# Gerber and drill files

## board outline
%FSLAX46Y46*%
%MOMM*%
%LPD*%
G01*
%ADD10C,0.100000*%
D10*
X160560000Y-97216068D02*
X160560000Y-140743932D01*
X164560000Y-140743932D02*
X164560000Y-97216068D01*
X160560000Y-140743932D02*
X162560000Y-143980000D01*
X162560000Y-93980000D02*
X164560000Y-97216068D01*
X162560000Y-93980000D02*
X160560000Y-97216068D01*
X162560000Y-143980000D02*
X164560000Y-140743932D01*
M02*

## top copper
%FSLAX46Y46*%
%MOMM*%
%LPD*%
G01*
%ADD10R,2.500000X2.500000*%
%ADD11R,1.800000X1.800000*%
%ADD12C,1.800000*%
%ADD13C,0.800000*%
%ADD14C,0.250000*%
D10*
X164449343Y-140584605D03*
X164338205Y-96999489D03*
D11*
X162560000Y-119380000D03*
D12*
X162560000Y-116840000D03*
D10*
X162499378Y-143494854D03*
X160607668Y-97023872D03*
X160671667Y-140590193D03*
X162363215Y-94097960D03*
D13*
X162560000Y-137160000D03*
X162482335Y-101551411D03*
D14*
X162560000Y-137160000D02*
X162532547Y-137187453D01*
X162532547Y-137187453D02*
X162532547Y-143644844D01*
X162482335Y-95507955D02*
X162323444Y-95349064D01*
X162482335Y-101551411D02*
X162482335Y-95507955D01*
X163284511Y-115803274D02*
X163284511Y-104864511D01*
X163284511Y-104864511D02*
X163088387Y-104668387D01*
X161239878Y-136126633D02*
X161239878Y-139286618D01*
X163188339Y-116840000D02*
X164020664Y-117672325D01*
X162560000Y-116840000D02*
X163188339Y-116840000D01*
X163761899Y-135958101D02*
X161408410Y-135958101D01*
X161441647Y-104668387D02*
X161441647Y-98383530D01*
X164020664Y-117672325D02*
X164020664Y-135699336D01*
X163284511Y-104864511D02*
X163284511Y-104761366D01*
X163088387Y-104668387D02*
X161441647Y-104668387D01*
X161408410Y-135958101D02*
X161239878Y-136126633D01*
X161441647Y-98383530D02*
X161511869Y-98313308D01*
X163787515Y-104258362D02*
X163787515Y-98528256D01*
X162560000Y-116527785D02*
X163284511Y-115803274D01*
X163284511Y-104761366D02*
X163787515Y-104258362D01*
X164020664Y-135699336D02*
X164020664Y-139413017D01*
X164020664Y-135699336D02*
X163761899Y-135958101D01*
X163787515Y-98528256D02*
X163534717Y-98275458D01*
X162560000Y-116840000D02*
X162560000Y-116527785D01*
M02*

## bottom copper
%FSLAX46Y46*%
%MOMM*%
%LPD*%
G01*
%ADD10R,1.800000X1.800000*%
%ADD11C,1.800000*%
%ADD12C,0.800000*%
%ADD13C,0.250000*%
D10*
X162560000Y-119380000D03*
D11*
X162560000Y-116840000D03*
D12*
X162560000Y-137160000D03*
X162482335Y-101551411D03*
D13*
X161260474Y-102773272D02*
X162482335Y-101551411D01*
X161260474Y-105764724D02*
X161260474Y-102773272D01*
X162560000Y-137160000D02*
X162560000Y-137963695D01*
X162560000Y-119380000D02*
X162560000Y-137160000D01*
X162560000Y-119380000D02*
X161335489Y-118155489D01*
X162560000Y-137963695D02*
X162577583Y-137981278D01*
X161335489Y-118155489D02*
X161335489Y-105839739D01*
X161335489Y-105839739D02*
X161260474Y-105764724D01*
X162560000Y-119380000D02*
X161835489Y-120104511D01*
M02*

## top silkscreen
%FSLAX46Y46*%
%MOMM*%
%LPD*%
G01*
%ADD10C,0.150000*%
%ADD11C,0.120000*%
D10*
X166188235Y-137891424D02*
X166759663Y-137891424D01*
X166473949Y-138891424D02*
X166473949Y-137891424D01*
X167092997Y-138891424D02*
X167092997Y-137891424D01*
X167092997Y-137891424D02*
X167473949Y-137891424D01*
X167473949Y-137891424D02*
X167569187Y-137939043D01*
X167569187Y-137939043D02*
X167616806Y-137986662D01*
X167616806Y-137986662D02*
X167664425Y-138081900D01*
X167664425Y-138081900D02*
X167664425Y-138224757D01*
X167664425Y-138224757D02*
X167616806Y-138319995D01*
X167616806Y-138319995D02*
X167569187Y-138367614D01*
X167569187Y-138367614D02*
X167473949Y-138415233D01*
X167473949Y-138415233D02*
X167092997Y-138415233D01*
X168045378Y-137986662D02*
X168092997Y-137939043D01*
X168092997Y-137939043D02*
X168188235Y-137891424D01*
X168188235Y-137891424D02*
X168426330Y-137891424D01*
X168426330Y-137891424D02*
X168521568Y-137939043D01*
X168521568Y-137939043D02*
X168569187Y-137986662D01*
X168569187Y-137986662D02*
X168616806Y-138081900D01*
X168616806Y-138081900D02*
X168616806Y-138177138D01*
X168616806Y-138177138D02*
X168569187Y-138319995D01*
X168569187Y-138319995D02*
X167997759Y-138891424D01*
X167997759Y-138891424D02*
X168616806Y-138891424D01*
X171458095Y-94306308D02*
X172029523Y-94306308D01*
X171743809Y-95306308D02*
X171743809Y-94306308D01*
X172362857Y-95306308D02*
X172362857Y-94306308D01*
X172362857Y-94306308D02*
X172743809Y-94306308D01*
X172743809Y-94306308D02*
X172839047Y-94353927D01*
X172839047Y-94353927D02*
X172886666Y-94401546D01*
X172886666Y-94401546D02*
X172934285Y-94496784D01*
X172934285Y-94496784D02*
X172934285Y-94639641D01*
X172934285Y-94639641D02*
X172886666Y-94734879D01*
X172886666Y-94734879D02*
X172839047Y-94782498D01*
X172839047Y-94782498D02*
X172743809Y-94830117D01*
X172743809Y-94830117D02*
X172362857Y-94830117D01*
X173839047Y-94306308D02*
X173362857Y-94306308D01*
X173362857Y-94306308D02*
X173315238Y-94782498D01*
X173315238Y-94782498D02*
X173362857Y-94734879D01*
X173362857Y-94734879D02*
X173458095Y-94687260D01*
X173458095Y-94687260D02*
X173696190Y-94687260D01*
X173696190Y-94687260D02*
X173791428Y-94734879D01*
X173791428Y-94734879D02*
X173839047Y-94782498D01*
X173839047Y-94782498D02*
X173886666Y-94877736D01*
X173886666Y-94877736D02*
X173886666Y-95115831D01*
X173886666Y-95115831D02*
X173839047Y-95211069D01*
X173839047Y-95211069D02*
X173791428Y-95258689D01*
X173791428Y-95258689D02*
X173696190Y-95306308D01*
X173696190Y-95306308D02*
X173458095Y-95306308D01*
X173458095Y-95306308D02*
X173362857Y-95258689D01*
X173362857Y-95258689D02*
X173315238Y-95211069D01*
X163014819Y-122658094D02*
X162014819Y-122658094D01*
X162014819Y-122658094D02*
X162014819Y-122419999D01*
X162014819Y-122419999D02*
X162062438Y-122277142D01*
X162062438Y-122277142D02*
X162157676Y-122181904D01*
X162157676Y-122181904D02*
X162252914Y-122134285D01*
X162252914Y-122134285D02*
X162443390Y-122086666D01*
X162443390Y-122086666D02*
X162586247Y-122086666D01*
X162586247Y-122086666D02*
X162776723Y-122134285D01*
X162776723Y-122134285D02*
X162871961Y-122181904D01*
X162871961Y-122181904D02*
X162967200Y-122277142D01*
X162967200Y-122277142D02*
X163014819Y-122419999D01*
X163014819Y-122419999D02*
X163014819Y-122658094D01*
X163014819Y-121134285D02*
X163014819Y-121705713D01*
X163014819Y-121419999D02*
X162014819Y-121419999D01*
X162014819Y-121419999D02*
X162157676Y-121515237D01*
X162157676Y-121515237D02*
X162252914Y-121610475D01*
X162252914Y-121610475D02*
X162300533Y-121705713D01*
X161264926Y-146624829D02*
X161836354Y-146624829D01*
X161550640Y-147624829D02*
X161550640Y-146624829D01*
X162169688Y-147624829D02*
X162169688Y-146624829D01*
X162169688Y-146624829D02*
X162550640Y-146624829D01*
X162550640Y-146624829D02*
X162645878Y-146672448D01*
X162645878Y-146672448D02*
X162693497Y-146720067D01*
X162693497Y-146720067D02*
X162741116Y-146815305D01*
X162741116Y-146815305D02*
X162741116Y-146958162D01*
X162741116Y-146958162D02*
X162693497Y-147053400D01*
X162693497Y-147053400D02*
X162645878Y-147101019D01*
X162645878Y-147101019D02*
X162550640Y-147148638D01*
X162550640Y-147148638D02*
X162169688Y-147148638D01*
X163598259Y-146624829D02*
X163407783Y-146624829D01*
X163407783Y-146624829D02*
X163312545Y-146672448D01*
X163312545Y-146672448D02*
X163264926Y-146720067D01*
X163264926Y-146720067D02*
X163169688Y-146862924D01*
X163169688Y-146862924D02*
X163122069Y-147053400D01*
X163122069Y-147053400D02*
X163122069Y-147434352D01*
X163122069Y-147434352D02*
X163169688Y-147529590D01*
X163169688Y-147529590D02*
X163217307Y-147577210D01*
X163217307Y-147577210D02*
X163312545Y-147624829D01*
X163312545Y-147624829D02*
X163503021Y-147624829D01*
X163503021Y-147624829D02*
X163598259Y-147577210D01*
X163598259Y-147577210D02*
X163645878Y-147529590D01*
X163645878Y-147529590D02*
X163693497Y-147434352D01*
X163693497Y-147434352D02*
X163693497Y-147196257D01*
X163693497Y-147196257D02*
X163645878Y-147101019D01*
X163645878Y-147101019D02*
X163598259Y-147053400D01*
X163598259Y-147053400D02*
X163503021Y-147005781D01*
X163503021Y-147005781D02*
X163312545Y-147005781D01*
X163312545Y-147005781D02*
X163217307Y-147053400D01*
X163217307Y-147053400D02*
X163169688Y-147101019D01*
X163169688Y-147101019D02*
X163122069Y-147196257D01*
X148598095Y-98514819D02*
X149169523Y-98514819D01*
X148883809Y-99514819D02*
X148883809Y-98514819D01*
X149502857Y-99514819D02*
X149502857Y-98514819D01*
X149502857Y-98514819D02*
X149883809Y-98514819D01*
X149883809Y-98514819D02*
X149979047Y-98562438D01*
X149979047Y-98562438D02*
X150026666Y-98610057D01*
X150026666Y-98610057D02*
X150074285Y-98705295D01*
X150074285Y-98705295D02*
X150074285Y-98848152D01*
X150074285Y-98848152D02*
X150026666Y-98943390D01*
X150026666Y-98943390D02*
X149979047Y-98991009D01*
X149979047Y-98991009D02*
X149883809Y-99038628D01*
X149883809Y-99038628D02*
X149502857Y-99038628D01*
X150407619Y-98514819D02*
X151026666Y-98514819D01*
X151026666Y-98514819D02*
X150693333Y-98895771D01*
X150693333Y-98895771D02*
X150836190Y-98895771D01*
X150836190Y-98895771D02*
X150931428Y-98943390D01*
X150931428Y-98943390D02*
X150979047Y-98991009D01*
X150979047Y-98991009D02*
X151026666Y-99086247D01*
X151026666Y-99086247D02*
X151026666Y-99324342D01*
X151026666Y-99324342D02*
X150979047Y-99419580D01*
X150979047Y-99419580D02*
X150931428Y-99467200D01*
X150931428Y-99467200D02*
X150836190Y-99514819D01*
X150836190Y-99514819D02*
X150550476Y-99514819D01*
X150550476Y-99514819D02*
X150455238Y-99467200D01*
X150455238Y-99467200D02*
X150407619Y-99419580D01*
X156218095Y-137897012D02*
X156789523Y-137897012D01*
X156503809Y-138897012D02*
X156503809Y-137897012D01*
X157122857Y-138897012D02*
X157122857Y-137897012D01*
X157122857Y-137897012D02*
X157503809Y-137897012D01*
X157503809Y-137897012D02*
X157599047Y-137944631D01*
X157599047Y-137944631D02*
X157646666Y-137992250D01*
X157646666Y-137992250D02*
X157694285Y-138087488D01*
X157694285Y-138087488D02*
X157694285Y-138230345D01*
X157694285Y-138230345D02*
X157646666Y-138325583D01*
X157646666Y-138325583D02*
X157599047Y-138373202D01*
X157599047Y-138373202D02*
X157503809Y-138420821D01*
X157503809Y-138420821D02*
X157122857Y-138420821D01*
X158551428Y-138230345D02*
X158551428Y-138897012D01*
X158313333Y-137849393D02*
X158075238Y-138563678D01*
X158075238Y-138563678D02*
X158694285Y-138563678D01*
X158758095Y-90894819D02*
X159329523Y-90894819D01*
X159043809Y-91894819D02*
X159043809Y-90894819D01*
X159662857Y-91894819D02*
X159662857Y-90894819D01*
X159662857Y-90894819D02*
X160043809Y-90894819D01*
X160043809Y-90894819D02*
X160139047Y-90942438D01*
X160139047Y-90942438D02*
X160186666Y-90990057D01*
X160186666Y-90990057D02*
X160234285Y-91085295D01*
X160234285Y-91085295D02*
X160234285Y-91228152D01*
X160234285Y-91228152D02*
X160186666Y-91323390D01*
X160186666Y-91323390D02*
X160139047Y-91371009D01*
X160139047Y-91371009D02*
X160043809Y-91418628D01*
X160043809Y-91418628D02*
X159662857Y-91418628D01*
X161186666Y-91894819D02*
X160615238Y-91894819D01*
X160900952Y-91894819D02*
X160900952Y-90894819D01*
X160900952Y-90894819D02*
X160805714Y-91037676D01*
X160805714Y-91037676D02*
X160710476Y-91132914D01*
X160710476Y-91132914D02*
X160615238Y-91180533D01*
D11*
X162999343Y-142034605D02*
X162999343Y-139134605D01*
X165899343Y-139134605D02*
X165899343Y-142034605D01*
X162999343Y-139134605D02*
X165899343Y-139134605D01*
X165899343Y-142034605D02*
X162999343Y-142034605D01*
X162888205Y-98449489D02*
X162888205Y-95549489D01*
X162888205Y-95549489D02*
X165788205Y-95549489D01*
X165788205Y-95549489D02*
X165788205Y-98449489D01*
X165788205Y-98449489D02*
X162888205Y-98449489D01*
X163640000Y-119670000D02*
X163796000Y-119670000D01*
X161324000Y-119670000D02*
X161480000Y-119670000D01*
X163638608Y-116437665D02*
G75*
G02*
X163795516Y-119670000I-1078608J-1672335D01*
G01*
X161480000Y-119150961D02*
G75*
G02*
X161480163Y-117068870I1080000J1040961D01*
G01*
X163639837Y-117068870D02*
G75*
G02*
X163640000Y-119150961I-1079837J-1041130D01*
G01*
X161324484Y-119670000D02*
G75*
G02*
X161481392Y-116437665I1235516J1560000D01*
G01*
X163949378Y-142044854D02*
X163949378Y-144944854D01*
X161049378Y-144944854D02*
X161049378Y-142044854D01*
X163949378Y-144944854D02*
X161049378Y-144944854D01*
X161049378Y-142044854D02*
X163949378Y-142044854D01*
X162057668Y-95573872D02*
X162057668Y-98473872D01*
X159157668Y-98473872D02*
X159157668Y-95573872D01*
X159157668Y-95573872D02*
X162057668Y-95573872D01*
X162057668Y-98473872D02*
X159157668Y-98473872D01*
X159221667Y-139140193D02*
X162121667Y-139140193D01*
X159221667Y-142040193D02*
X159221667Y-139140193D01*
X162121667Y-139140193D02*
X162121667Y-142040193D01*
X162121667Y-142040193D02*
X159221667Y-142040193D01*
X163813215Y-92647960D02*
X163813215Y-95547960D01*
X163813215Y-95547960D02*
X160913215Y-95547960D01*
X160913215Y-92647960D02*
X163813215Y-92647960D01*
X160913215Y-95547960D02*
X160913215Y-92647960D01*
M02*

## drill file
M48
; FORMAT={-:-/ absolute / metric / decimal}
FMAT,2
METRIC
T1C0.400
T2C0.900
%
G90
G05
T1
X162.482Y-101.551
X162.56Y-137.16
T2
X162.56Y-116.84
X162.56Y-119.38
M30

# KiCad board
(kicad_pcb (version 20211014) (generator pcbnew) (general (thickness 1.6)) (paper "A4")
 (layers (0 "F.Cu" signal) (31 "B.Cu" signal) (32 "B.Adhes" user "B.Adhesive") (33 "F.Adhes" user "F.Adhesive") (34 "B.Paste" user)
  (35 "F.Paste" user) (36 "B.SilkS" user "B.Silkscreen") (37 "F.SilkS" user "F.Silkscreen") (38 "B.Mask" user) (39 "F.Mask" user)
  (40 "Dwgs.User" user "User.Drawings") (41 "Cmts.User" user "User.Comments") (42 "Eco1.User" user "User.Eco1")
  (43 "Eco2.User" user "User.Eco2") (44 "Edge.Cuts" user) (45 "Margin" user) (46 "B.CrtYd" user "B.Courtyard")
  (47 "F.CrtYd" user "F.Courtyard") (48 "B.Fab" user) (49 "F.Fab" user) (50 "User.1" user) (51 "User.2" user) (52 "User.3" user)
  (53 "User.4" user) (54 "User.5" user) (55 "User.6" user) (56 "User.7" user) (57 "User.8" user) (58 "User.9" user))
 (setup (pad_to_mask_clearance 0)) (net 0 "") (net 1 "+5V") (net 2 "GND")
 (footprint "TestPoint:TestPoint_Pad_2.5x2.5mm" (layer "F.Cu") (at 164.449343 140.584605)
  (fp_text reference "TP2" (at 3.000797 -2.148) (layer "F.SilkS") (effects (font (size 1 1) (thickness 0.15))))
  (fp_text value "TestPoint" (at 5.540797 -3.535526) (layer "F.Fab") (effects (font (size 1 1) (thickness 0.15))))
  (fp_line (start -1.45 1.45) (end -1.45 -1.45) (layer "F.SilkS") (width 0.12))
  (fp_line (start 1.45 -1.45) (end 1.45 1.45) (layer "F.SilkS") (width 0.12))
  (fp_line (start -1.45 -1.45) (end 1.45 -1.45) (layer "F.SilkS") (width 0.12))
  (fp_line (start 1.45 1.45) (end -1.45 1.45) (layer "F.SilkS") (width 0.12))
  (pad "1" smd rect (at 0 0) (size 2.5 2.5) (layers "F.Cu" "F.Mask") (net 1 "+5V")))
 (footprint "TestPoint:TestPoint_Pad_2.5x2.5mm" (layer "F.Cu") (at 164.338205 96.999489)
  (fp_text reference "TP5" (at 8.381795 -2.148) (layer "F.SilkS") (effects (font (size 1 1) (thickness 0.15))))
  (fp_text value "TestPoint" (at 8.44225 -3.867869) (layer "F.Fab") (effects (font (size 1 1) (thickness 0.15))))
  (fp_line (start -1.45 1.45) (end -1.45 -1.45) (layer "F.SilkS") (width 0.12))
  (fp_line (start -1.45 -1.45) (end 1.45 -1.45) (layer "F.SilkS") (width 0.12))
  (fp_line (start 1.45 -1.45) (end 1.45 1.45) (layer "F.SilkS") (width 0.12))
  (fp_line (start 1.45 1.45) (end -1.45 1.45) (layer "F.SilkS") (width 0.12))
  (pad "1" smd rect (at 0 0) (size 2.5 2.5) (layers "F.Cu" "F.Mask") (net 1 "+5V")))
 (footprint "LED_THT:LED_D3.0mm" (layer "F.Cu") (at 162.56 119.38 90)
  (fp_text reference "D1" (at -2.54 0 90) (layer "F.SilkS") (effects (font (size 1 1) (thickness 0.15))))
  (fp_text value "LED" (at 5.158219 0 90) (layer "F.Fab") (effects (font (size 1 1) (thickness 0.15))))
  (fp_line (start -0.29 1.08) (end -0.29 1.236) (layer "F.SilkS") (width 0.12))
  (fp_line (start -0.29 -1.236) (end -0.29 -1.08) (layer "F.SilkS") (width 0.12))
  (fp_arc (start 2.942335 1.078608) (mid 1.366487 1.987659) (end -0.29 1.235516) (layer "F.SilkS") (width 0.12))
  (fp_arc (start 0.229039 -1.08) (mid 1.270117 -1.5) (end 2.31113 -1.079837) (layer "F.SilkS") (width 0.12))
  (fp_arc (start 2.31113 1.079837) (mid 1.270117 1.5) (end 0.229039 1.08) (layer "F.SilkS") (width 0.12))
  (fp_arc (start -0.29 -1.235516) (mid 1.366487 -1.987659) (end 2.942335 -1.078608) (layer "F.SilkS") (width 0.12))
  (pad "1" thru_hole rect (at 0 0 90) (size 1.8 1.8) (drill 0.9) (layers *.Cu *.Mask) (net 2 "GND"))
  (pad "2" thru_hole circle (at 2.54 0 90) (size 1.8 1.8) (drill 0.9) (layers *.Cu *.Mask) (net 1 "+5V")))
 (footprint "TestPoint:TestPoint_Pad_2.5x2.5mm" (layer "F.Cu") (at 162.499378 143.494854)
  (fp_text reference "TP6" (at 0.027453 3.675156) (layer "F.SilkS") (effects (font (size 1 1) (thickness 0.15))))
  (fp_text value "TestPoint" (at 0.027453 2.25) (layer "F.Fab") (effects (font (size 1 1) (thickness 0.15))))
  (fp_line (start 1.45 -1.45) (end 1.45 1.45) (layer "F.SilkS") (width 0.12))
  (fp_line (start -1.45 1.45) (end -1.45 -1.45) (layer "F.SilkS") (width 0.12))
  (fp_line (start 1.45 1.45) (end -1.45 1.45) (layer "F.SilkS") (width 0.12))
  (fp_line (start -1.45 -1.45) (end 1.45 -1.45) (layer "F.SilkS") (width 0.12))
  (pad "1" smd rect (at 0 0) (size 2.5 2.5) (layers "F.Cu" "F.Mask") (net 2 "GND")))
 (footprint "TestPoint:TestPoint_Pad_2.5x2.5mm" (layer "F.Cu") (at 160.607668 97.023872)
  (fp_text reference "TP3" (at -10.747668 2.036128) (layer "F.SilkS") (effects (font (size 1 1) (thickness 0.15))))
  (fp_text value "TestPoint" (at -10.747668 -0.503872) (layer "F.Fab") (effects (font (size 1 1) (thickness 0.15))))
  (fp_line (start 1.45 -1.45) (end 1.45 1.45) (layer "F.SilkS") (width 0.12))
  (fp_line (start -1.45 1.45) (end -1.45 -1.45) (layer "F.SilkS") (width 0.12))
  (fp_line (start -1.45 -1.45) (end 1.45 -1.45) (layer "F.SilkS") (width 0.12))
  (fp_line (start 1.45 1.45) (end -1.45 1.45) (layer "F.SilkS") (width 0.12))
  (pad "1" smd rect (at 0 0) (size 2.5 2.5) (layers "F.Cu" "F.Mask") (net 1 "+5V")))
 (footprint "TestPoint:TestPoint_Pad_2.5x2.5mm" (layer "F.Cu") (at 160.671667 140.590193)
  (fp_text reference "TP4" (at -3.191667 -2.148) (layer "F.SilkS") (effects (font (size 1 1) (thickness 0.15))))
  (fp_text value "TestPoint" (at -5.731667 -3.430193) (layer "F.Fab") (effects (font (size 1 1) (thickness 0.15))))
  (fp_line (start -1.45 -1.45) (end 1.45 -1.45) (layer "F.SilkS") (width 0.12))
  (fp_line (start -1.45 1.45) (end -1.45 -1.45) (layer "F.SilkS") (width 0.12))
  (fp_line (start 1.45 -1.45) (end 1.45 1.45) (layer "F.SilkS") (width 0.12))
  (fp_line (start 1.45 1.45) (end -1.45 1.45) (layer "F.SilkS") (width 0.12))
  (pad "1" smd rect (at 0 0) (size 2.5 2.5) (layers "F.Cu" "F.Mask") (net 1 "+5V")))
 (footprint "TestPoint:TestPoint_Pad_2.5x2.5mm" (layer "F.Cu") (at 162.363215 94.09796)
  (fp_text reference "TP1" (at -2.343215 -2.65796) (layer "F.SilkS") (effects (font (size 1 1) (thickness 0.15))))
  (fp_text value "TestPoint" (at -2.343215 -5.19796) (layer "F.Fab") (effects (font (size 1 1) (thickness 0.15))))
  (fp_line (start 1.45 -1.45) (end 1.45 1.45) (layer "F.SilkS") (width 0.12))
  (fp_line (start 1.45 1.45) (end -1.45 1.45) (layer "F.SilkS") (width 0.12))
  (fp_line (start -1.45 -1.45) (end 1.45 -1.45) (layer "F.SilkS") (width 0.12))
  (fp_line (start -1.45 1.45) (end -1.45 -1.45) (layer "F.SilkS") (width 0.12))
  (pad "1" smd rect (at 0 0) (size 2.5 2.5) (layers "F.Cu" "F.Mask") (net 2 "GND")))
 (gr_line (start 160.56 97.216068) (end 160.56 140.743932) (layer "Edge.Cuts") (width 0.1))
 (gr_line (start 164.56 140.743932) (end 164.56 97.216068) (layer "Edge.Cuts") (width 0.1))
 (gr_line (start 160.56 140.743932) (end 162.56 143.98) (layer "Edge.Cuts") (width 0.1))
 (gr_line (start 162.56 93.98) (end 164.56 97.216068) (layer "Edge.Cuts") (width 0.1))
 (gr_line (start 162.56 93.98) (end 160.56 97.216068) (layer "Edge.Cuts") (width 0.1))
 (gr_line (start 162.56 143.98) (end 164.56 140.743932) (layer "Edge.Cuts") (width 0.1))
 (segment (start 162.56 137.16) (end 162.532547 137.187453) (width 0.25) (layer "F.Cu") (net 2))
 (segment (start 162.532547 137.187453) (end 162.532547 143.644844) (width 0.25) (layer "F.Cu") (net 2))
 (segment (start 162.482335 95.507955) (end 162.323444 95.349064) (width 0.25) (layer "F.Cu") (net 2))
 (segment (start 162.482335 101.551411) (end 162.482335 95.507955) (width 0.25) (layer "F.Cu") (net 2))
 (via (at 162.56 137.16) (size 0.8) (drill 0.4) (layers "F.Cu" "B.Cu") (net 2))
 (via (at 162.482335 101.551411) (size 0.8) (drill 0.4) (layers "F.Cu" "B.Cu") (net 2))
 (segment (start 161.260474 102.773272) (end 162.482335 101.551411) (width 0.25) (layer "B.Cu") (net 2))
 (segment (start 161.260474 105.764724) (end 161.260474 102.773272) (width 0.25) (layer "B.Cu") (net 2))
 (segment (start 162.56 137.16) (end 162.56 137.963695) (width 0.25) (layer "B.Cu") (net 2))
 (segment (start 162.56 119.38) (end 162.56 137.16) (width 0.25) (layer "B.Cu") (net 2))
 (segment (start 162.56 119.38) (end 161.335489 118.155489) (width 0.25) (layer "B.Cu") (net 2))
 (segment (start 162.56 137.963695) (end 162.577583 137.981278) (width 0.25) (layer "B.Cu") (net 2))
 (segment (start 161.335489 118.155489) (end 161.335489 105.839739) (width 0.25) (layer "B.Cu") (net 2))
 (segment (start 161.335489 105.839739) (end 161.260474 105.764724) (width 0.25) (layer "B.Cu") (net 2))
 (segment (start 162.56 119.38) (end 161.835489 120.104511) (width 0.25) (layer "B.Cu") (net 2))
 (segment (start 163.284511 115.803274) (end 163.284511 104.864511) (width 0.25) (layer "F.Cu") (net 1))
 (segment (start 163.284511 104.864511) (end 163.088387 104.668387) (width 0.25) (layer "F.Cu") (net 1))
 (segment (start 161.239878 136.126633) (end 161.239878 139.286618) (width 0.25) (layer "F.Cu") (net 1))
 (segment (start 163.188339 116.84) (end 164.020664 117.672325) (width 0.25) (layer "F.Cu") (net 1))
 (segment (start 162.56 116.84) (end 163.188339 116.84) (width 0.25) (layer "F.Cu") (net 1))
 (segment (start 163.761899 135.958101) (end 161.40841 135.958101) (width 0.25) (layer "F.Cu") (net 1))
 (segment (start 161.441647 104.668387) (end 161.441647 98.38353) (width 0.25) (layer "F.Cu") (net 1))
 (segment (start 164.020664 117.672325) (end 164.020664 135.699336) (width 0.25) (layer "F.Cu") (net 1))
 (segment (start 163.284511 104.864511) (end 163.284511 104.761366) (width 0.25) (layer "F.Cu") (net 1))
 (segment (start 163.088387 104.668387) (end 161.441647 104.668387) (width 0.25) (layer "F.Cu") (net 1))
 (segment (start 161.40841 135.958101) (end 161.239878 136.126633) (width 0.25) (layer "F.Cu") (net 1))
 (segment (start 161.441647 98.38353) (end 161.511869 98.313308) (width 0.25) (layer "F.Cu") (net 1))
 (segment (start 163.787515 104.258362) (end 163.787515 98.528256) (width 0.25) (layer "F.Cu") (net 1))
 (segment (start 162.56 116.527785) (end 163.284511 115.803274) (width 0.25) (layer "F.Cu") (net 1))
 (segment (start 163.284511 104.761366) (end 163.787515 104.258362) (width 0.25) (layer "F.Cu") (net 1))
 (segment (start 164.020664 135.699336) (end 164.020664 139.413017) (width 0.25) (layer "F.Cu") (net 1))
 (segment (start 164.020664 135.699336) (end 163.761899 135.958101) (width 0.25) (layer "F.Cu") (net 1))
 (segment (start 163.787515 98.528256) (end 163.534717 98.275458) (width 0.25) (layer "F.Cu") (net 1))
 (segment (start 162.56 116.84) (end 162.56 116.527785) (width 0.25) (layer "F.Cu") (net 1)))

